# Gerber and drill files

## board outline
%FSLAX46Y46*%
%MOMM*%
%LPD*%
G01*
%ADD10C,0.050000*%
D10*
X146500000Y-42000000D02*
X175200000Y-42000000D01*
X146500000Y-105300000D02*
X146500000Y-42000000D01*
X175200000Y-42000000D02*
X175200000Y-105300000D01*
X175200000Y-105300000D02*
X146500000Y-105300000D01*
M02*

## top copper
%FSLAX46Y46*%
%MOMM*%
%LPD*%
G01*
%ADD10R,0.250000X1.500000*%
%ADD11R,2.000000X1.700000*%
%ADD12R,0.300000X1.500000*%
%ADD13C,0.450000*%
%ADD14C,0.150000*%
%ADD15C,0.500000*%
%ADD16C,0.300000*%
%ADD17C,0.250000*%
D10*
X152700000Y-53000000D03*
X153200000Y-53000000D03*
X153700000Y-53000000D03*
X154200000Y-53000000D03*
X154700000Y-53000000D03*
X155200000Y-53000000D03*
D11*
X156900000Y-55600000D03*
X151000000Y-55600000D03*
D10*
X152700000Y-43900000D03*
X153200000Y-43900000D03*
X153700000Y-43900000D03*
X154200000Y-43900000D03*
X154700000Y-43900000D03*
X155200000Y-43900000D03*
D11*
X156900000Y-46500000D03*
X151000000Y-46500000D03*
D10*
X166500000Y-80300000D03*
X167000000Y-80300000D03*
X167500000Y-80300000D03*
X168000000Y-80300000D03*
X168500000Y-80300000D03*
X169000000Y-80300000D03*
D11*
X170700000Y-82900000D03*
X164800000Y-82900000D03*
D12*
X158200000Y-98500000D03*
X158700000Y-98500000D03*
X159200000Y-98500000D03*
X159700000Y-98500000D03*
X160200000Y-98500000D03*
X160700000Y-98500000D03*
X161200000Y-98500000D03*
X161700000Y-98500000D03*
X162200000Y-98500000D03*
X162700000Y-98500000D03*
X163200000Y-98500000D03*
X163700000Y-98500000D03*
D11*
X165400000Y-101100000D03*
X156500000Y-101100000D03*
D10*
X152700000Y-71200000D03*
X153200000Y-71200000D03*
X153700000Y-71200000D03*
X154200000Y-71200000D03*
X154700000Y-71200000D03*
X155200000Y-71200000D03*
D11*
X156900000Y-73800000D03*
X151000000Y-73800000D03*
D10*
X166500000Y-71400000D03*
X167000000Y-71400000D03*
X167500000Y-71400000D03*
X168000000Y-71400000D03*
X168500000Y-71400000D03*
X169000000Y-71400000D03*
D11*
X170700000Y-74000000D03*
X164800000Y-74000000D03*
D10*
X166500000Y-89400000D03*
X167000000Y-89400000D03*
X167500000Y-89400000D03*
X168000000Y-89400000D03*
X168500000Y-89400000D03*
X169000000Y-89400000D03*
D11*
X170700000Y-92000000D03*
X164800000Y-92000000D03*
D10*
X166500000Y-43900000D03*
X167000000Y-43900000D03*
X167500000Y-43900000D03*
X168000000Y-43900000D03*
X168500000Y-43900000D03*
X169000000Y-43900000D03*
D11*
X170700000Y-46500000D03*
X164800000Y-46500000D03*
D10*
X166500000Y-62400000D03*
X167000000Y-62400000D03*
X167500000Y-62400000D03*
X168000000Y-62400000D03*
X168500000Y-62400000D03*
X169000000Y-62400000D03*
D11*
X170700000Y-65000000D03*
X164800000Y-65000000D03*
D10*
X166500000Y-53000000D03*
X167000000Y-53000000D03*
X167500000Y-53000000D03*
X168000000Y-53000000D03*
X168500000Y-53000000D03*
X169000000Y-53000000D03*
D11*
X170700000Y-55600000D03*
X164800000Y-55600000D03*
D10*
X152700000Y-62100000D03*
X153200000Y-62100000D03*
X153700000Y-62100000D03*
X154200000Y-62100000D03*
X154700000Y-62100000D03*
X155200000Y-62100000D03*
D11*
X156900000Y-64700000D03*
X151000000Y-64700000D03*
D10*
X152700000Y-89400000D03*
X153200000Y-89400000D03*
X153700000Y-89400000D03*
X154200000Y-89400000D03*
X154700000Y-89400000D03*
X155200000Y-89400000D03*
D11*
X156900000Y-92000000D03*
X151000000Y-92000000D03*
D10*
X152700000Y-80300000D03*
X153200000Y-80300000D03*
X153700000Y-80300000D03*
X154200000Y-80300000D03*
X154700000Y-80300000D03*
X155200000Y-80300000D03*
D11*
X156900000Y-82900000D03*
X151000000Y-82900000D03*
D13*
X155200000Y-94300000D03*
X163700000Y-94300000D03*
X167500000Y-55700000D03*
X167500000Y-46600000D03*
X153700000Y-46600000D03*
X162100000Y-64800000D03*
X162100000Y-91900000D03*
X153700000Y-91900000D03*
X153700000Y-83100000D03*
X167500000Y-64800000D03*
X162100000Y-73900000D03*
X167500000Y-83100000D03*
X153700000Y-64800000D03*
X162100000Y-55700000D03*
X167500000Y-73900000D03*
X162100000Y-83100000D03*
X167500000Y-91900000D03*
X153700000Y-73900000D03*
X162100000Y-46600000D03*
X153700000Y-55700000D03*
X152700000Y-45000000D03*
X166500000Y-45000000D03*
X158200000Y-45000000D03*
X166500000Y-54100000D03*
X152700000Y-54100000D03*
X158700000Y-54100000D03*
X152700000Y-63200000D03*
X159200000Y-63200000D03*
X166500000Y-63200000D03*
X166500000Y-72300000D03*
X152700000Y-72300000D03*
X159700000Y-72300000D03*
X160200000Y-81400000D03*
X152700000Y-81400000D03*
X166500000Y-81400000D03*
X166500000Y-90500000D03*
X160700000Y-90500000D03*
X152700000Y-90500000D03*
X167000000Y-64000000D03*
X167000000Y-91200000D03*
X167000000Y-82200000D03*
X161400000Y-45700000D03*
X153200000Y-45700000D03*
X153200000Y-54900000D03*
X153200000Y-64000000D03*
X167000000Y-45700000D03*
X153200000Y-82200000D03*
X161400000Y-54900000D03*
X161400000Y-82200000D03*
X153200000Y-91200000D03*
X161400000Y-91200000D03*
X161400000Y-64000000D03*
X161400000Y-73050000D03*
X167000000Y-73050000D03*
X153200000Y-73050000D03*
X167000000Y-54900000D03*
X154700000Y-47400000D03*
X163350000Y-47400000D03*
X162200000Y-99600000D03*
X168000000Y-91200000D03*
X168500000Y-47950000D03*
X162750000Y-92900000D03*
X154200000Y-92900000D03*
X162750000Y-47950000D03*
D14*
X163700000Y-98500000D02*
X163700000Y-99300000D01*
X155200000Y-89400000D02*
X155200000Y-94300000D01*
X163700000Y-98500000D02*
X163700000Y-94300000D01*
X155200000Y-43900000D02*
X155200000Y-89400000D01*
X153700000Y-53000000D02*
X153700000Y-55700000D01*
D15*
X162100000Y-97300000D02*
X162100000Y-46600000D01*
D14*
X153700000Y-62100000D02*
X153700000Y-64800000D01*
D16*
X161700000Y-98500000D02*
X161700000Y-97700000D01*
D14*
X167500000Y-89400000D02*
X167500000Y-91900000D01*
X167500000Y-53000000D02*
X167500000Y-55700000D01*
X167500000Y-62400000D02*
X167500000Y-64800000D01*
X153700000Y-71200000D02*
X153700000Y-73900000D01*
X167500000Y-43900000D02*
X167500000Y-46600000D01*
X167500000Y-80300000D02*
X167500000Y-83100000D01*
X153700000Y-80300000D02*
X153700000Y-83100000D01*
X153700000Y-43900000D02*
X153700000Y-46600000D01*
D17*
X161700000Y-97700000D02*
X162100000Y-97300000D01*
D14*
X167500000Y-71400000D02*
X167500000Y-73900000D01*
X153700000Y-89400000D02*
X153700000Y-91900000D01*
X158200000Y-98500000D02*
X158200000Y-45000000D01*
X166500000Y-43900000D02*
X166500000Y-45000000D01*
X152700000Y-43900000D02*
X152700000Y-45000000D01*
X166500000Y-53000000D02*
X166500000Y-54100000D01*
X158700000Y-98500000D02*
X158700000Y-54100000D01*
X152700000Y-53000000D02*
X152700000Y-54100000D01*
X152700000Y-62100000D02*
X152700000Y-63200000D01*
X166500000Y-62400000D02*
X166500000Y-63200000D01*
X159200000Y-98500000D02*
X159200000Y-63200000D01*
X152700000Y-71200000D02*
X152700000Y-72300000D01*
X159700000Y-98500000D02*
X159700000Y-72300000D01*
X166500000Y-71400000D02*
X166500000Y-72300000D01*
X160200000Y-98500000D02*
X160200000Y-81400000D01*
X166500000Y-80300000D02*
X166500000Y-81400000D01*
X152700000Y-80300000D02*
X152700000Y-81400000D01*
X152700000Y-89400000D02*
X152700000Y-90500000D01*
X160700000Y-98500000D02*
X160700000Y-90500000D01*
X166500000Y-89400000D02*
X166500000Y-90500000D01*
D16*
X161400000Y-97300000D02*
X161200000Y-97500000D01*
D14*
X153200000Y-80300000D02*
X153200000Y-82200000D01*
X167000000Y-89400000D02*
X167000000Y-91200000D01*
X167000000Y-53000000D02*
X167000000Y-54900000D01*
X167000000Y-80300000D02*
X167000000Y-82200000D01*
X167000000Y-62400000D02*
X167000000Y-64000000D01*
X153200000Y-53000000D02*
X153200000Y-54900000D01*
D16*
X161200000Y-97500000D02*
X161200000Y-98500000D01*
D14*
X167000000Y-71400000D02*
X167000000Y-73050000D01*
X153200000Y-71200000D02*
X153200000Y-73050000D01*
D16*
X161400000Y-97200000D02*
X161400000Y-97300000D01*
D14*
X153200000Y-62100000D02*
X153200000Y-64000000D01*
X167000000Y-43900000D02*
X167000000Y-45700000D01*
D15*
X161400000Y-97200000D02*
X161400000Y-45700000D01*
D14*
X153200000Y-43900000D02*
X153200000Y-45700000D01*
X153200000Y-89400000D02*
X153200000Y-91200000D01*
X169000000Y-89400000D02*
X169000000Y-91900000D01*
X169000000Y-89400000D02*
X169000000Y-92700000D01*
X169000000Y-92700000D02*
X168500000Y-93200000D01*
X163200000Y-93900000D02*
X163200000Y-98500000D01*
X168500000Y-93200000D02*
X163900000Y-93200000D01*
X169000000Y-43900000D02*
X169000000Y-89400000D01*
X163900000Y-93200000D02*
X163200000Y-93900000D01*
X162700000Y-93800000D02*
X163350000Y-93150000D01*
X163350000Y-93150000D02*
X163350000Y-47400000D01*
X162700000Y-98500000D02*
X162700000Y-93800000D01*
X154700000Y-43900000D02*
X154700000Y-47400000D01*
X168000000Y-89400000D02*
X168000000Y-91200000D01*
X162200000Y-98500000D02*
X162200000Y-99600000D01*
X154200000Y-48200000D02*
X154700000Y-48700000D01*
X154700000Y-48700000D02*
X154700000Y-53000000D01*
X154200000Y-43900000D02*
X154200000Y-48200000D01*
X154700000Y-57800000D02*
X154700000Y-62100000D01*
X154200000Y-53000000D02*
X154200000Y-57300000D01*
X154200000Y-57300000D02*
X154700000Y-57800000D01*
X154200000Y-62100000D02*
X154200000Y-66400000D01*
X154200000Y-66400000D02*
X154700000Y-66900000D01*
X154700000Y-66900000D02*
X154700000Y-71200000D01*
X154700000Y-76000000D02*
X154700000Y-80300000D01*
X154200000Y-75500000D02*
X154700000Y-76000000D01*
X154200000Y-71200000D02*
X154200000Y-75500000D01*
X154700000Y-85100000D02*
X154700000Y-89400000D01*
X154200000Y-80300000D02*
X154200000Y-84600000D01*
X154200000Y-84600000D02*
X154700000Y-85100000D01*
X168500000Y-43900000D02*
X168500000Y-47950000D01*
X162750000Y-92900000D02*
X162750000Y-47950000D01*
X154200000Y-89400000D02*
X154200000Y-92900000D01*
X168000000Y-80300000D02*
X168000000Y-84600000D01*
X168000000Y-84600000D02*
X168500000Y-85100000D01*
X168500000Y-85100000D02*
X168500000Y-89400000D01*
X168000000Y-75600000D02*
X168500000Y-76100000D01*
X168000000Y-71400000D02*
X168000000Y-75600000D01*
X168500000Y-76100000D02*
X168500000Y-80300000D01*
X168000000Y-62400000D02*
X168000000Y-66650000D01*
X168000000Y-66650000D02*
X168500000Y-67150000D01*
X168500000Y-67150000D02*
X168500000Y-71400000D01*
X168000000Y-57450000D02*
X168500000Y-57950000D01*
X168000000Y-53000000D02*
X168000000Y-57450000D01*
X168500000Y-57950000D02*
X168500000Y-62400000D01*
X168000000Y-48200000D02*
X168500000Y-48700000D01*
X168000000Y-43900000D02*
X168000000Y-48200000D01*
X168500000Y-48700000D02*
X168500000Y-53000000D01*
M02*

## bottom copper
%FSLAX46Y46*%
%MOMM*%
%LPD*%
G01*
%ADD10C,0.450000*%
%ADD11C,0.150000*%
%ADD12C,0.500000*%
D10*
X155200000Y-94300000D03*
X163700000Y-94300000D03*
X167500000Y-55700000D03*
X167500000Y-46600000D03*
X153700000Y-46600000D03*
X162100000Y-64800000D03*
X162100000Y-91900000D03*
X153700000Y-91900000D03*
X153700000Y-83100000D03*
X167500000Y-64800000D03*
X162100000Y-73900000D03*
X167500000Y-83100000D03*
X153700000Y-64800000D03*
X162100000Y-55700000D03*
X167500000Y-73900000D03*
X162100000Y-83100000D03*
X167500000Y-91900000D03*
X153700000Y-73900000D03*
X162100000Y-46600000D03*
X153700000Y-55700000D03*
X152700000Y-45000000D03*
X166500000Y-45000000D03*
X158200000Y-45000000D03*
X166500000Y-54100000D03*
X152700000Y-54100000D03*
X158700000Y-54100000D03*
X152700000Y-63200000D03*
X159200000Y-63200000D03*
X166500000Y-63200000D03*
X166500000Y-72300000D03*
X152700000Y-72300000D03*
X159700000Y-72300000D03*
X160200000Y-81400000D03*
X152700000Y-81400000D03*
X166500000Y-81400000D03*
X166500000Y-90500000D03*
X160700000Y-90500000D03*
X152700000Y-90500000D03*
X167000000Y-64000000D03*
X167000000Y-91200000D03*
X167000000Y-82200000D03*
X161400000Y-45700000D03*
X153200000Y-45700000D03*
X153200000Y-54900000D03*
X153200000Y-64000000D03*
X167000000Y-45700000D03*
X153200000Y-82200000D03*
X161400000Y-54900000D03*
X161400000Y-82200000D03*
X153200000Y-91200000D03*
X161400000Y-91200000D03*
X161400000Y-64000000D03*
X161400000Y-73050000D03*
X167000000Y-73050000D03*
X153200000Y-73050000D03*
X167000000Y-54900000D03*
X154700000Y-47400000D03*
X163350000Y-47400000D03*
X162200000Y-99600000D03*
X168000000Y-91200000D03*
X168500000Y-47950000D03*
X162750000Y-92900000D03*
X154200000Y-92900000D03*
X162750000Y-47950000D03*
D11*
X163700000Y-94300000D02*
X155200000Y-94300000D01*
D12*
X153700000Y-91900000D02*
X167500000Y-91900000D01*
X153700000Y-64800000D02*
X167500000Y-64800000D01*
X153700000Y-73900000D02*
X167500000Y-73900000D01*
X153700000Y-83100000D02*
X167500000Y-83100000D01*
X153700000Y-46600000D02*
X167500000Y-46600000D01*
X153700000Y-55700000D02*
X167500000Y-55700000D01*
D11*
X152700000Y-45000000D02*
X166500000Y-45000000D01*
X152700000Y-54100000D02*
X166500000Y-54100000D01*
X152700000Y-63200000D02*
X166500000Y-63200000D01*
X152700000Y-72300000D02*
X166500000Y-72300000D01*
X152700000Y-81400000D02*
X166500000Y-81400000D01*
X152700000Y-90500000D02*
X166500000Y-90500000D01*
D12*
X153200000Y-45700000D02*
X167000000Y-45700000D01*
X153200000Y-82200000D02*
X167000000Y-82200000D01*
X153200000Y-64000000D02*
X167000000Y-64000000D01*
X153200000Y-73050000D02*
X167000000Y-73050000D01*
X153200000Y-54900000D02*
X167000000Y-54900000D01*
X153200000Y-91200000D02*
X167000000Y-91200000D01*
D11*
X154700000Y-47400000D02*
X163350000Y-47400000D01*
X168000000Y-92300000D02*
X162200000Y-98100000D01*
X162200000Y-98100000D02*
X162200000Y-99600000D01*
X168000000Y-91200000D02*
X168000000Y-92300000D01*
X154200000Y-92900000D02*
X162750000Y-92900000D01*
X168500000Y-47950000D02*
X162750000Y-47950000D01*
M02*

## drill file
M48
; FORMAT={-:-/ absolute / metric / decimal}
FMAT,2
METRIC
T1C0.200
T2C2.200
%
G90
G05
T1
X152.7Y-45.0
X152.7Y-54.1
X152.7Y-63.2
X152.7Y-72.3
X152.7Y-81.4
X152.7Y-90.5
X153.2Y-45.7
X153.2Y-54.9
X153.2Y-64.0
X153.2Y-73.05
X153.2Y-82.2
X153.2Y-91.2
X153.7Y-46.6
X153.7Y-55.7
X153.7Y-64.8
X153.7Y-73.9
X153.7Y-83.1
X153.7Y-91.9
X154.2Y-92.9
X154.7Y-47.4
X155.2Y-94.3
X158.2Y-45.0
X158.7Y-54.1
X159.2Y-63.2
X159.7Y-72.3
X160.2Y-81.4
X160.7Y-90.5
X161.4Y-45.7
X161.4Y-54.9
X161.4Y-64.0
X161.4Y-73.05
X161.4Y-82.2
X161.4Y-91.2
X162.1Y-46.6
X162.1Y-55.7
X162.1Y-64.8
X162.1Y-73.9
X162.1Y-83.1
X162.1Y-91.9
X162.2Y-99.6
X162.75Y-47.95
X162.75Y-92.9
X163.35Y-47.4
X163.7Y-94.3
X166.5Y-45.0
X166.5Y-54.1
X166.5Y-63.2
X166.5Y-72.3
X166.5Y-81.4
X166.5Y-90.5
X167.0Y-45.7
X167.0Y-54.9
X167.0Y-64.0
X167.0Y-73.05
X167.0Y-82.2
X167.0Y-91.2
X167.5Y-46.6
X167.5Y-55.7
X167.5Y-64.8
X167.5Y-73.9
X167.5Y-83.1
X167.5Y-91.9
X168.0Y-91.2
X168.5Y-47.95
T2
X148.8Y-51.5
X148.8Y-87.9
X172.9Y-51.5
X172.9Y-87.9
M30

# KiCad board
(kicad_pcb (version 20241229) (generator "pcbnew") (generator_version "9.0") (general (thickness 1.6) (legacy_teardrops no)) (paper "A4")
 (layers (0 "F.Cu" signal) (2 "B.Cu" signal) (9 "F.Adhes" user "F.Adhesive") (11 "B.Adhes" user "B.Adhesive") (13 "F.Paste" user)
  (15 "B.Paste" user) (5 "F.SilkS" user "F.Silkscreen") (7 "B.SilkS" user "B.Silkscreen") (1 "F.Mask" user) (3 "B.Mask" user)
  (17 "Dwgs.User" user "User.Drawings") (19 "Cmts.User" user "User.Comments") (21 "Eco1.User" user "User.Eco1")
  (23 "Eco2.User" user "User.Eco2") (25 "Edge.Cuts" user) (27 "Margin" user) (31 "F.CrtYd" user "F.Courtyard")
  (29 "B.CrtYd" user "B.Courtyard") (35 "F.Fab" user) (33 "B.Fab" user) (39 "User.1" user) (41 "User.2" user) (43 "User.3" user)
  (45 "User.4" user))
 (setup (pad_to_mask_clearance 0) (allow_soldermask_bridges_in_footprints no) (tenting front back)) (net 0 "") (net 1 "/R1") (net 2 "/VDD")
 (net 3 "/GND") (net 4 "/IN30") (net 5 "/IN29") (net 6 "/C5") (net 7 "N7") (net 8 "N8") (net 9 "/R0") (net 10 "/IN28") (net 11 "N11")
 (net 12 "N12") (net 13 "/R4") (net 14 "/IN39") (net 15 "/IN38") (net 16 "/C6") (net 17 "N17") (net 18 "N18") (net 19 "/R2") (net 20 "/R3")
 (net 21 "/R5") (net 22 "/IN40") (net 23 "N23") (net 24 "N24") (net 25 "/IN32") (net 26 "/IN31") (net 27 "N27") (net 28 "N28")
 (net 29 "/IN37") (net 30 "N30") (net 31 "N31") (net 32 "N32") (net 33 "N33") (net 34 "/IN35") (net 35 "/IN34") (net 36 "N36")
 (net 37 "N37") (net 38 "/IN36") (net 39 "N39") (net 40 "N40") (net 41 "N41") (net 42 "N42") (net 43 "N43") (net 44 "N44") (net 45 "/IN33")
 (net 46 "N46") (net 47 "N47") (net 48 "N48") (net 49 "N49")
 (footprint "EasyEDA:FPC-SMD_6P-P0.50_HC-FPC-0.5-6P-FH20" (layer "F.Cu") (at 153.95 54.3)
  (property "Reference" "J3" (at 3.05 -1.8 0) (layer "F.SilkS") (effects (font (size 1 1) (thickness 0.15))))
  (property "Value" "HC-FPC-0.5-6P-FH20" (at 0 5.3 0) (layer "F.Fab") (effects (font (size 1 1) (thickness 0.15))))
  (pad "1" smd rect (at -1.25 -1.3) (size 0.25 1.5) (layers "F.Cu" "F.Mask" "F.Paste") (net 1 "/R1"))
  (pad "2" smd rect (at -0.75 -1.3) (size 0.25 1.5) (layers "F.Cu" "F.Mask" "F.Paste") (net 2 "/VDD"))
  (pad "3" smd rect (at -0.25 -1.3) (size 0.25 1.5) (layers "F.Cu" "F.Mask" "F.Paste") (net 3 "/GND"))
  (pad "4" smd rect (at 0.25 -1.3) (size 0.25 1.5) (layers "F.Cu" "F.Mask" "F.Paste") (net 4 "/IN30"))
  (pad "5" smd rect (at 0.75 -1.3) (size 0.25 1.5) (layers "F.Cu" "F.Mask" "F.Paste") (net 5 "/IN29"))
  (pad "6" smd rect (at 1.25 -1.3) (size 0.25 1.5) (layers "F.Cu" "F.Mask" "F.Paste") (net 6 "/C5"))
  (pad "7" smd rect (at 2.95 1.3) (size 2 1.7) (layers "F.Cu" "F.Mask" "F.Paste") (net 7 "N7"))
  (pad "8" smd rect (at -2.95 1.3) (size 2 1.7) (layers "F.Cu" "F.Mask" "F.Paste") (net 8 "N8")))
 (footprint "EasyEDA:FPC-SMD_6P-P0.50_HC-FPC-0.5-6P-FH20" (layer "F.Cu") (at 153.95 45.2)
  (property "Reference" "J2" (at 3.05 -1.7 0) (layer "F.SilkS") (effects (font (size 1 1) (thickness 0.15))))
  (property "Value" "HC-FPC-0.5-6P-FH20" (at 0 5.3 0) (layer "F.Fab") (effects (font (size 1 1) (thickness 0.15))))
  (pad "1" smd rect (at -1.25 -1.3) (size 0.25 1.5) (layers "F.Cu" "F.Mask" "F.Paste") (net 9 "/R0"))
  (pad "2" smd rect (at -0.75 -1.3) (size 0.25 1.5) (layers "F.Cu" "F.Mask" "F.Paste") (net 2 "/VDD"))
  (pad "3" smd rect (at -0.25 -1.3) (size 0.25 1.5) (layers "F.Cu" "F.Mask" "F.Paste") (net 3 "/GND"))
  (pad "4" smd rect (at 0.25 -1.3) (size 0.25 1.5) (layers "F.Cu" "F.Mask" "F.Paste") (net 5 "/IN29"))
  (pad "5" smd rect (at 0.75 -1.3) (size 0.25 1.5) (layers "F.Cu" "F.Mask" "F.Paste") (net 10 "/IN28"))
  (pad "6" smd rect (at 1.25 -1.3) (size 0.25 1.5) (layers "F.Cu" "F.Mask" "F.Paste") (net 6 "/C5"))
  (pad "7" smd rect (at 2.95 1.3) (size 2 1.7) (layers "F.Cu" "F.Mask" "F.Paste") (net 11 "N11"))
  (pad "8" smd rect (at -2.95 1.3) (size 2 1.7) (layers "F.Cu" "F.Mask" "F.Paste") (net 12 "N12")))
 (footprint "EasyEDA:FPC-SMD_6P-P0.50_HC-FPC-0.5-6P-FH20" (layer "F.Cu") (at 167.75 81.6)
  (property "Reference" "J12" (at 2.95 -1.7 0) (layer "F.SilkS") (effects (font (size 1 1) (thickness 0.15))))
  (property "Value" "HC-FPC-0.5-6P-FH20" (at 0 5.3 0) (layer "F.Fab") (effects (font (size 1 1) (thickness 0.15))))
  (pad "1" smd rect (at -1.25 -1.3) (size 0.25 1.5) (layers "F.Cu" "F.Mask" "F.Paste") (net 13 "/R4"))
  (pad "2" smd rect (at -0.75 -1.3) (size 0.25 1.5) (layers "F.Cu" "F.Mask" "F.Paste") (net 2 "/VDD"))
  (pad "3" smd rect (at -0.25 -1.3) (size 0.25 1.5) (layers "F.Cu" "F.Mask" "F.Paste") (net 3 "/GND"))
  (pad "4" smd rect (at 0.25 -1.3) (size 0.25 1.5) (layers "F.Cu" "F.Mask" "F.Paste") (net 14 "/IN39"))
  (pad "5" smd rect (at 0.75 -1.3) (size 0.25 1.5) (layers "F.Cu" "F.Mask" "F.Paste") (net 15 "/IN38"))
  (pad "6" smd rect (at 1.25 -1.3) (size 0.25 1.5) (layers "F.Cu" "F.Mask" "F.Paste") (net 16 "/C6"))
  (pad "7" smd rect (at 2.95 1.3) (size 2 1.7) (layers "F.Cu" "F.Mask" "F.Paste") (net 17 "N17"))
  (pad "8" smd rect (at -2.95 1.3) (size 2 1.7) (layers "F.Cu" "F.Mask" "F.Paste") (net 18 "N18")))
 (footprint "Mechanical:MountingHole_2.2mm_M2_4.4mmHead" (layer "F.Cu") (at 148.8 87.9)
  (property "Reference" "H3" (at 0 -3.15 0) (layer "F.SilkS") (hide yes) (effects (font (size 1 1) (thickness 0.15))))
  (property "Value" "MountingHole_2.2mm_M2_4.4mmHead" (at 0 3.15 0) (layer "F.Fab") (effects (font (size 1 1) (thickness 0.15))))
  (pad "" np_thru_hole circle (at 0 0) (size 2.2 2.2) (drill 2.2) (layers "*.Cu" "*.Mask")))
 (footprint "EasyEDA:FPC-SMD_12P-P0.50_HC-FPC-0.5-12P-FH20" (layer "F.Cu") (at 160.95 99.8)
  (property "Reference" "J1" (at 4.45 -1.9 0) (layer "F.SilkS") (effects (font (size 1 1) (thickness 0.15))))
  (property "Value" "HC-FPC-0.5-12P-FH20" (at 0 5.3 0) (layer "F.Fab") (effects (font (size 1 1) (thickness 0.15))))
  (pad "1" smd rect (at -2.75 -1.3) (size 0.3 1.5) (layers "F.Cu" "F.Mask" "F.Paste") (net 9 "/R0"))
  (pad "2" smd rect (at -2.25 -1.3) (size 0.3 1.5) (layers "F.Cu" "F.Mask" "F.Paste") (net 1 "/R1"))
  (pad "3" smd rect (at -1.75 -1.3) (size 0.3 1.5) (layers "F.Cu" "F.Mask" "F.Paste") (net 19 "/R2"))
  (pad "4" smd rect (at -1.25 -1.3) (size 0.3 1.5) (layers "F.Cu" "F.Mask" "F.Paste") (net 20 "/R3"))
  (pad "5" smd rect (at -0.75 -1.3) (size 0.3 1.5) (layers "F.Cu" "F.Mask" "F.Paste") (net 13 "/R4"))
  (pad "6" smd rect (at -0.25 -1.3) (size 0.3 1.5) (layers "F.Cu" "F.Mask" "F.Paste") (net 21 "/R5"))
  (pad "7" smd rect (at 0.25 -1.3) (size 0.3 1.5) (layers "F.Cu" "F.Mask" "F.Paste") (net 2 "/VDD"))
  (pad "8" smd rect (at 0.75 -1.3) (size 0.3 1.5) (layers "F.Cu" "F.Mask" "F.Paste") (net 3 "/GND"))
  (pad "9" smd rect (at 1.25 -1.3) (size 0.3 1.5) (layers "F.Cu" "F.Mask" "F.Paste") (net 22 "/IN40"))
  (pad "10" smd rect (at 1.75 -1.3) (size 0.3 1.5) (layers "F.Cu" "F.Mask" "F.Paste") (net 10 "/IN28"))
  (pad "11" smd rect (at 2.25 -1.3) (size 0.3 1.5) (layers "F.Cu" "F.Mask" "F.Paste") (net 16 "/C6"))
  (pad "12" smd rect (at 2.75 -1.3) (size 0.3 1.5) (layers "F.Cu" "F.Mask" "F.Paste") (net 6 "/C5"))
  (pad "13" smd rect (at 4.45 1.3) (size 2 1.7) (layers "F.Cu" "F.Mask" "F.Paste") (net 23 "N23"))
  (pad "14" smd rect (at -4.45 1.3) (size 2 1.7) (layers "F.Cu" "F.Mask" "F.Paste") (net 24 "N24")))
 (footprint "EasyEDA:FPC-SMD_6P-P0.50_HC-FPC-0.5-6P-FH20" (layer "F.Cu") (at 153.95 72.5)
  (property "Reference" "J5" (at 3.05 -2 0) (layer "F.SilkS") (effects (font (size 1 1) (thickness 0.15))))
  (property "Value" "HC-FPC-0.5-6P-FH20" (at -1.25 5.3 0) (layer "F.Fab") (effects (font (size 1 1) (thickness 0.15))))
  (pad "1" smd rect (at -1.25 -1.3) (size 0.25 1.5) (layers "F.Cu" "F.Mask" "F.Paste") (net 20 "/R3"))
  (pad "2" smd rect (at -0.75 -1.3) (size 0.25 1.5) (layers "F.Cu" "F.Mask" "F.Paste") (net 2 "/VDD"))
  (pad "3" smd rect (at -0.25 -1.3) (size 0.25 1.5) (layers "F.Cu" "F.Mask" "F.Paste") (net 3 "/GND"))
  (pad "4" smd rect (at 0.25 -1.3) (size 0.25 1.5) (layers "F.Cu" "F.Mask" "F.Paste") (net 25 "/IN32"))
  (pad "5" smd rect (at 0.75 -1.3) (size 0.25 1.5) (layers "F.Cu" "F.Mask" "F.Paste") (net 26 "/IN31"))
  (pad "6" smd rect (at 1.25 -1.3) (size 0.25 1.5) (layers "F.Cu" "F.Mask" "F.Paste") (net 6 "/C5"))
  (pad "7" smd rect (at 2.95 1.3) (size 2 1.7) (layers "F.Cu" "F.Mask" "F.Paste") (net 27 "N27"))
  (pad "8" smd rect (at -2.95 1.3) (size 2 1.7) (layers "F.Cu" "F.Mask" "F.Paste") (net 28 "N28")))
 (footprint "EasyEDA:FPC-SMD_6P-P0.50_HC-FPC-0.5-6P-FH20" (layer "F.Cu") (at 167.75 72.7)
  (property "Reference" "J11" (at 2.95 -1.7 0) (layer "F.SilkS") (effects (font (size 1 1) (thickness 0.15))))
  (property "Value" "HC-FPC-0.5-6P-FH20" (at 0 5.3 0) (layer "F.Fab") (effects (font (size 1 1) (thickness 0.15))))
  (pad "1" smd rect (at -1.25 -1.3) (size 0.25 1.5) (layers "F.Cu" "F.Mask" "F.Paste") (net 20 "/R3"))
  (pad "2" smd rect (at -0.75 -1.3) (size 0.25 1.5) (layers "F.Cu" "F.Mask" "F.Paste") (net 2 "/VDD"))
  (pad "3" smd rect (at -0.25 -1.3) (size 0.25 1.5) (layers "F.Cu" "F.Mask" "F.Paste") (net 3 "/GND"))
  (pad "4" smd rect (at 0.25 -1.3) (size 0.25 1.5) (layers "F.Cu" "F.Mask" "F.Paste") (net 15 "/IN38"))
  (pad "5" smd rect (at 0.75 -1.3) (size 0.25 1.5) (layers "F.Cu" "F.Mask" "F.Paste") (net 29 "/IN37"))
  (pad "6" smd rect (at 1.25 -1.3) (size 0.25 1.5) (layers "F.Cu" "F.Mask" "F.Paste") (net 16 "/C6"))
  (pad "7" smd rect (at 2.95 1.3) (size 2 1.7) (layers "F.Cu" "F.Mask" "F.Paste") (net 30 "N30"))
  (pad "8" smd rect (at -2.95 1.3) (size 2 1.7) (layers "F.Cu" "F.Mask" "F.Paste") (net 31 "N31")))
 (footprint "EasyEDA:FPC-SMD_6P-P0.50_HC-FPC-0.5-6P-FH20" (layer "F.Cu") (at 167.75 90.7)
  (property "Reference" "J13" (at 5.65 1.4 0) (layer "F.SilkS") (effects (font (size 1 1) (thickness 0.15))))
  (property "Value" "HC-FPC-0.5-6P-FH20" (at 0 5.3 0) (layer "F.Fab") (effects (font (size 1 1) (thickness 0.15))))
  (pad "1" smd rect (at -1.25 -1.3) (size 0.25 1.5) (layers "F.Cu" "F.Mask" "F.Paste") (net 21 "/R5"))
  (pad "2" smd rect (at -0.75 -1.3) (size 0.25 1.5) (layers "F.Cu" "F.Mask" "F.Paste") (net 2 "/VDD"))
  (pad "3" smd rect (at -0.25 -1.3) (size 0.25 1.5) (layers "F.Cu" "F.Mask" "F.Paste") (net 3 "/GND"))
  (pad "4" smd rect (at 0.25 -1.3) (size 0.25 1.5) (layers "F.Cu" "F.Mask" "F.Paste") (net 22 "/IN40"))
  (pad "5" smd rect (at 0.75 -1.3) (size 0.25 1.5) (layers "F.Cu" "F.Mask" "F.Paste") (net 14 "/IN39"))
  (pad "6" smd rect (at 1.25 -1.3) (size 0.25 1.5) (layers "F.Cu" "F.Mask" "F.Paste") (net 16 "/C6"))
  (pad "7" smd rect (at 2.95 1.3) (size 2 1.7) (layers "F.Cu" "F.Mask" "F.Paste") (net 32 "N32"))
  (pad "8" smd rect (at -2.95 1.3) (size 2 1.7) (layers "F.Cu" "F.Mask" "F.Paste") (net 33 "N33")))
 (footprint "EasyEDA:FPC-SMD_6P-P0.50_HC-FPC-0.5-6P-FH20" (layer "F.Cu") (at 167.75 45.2)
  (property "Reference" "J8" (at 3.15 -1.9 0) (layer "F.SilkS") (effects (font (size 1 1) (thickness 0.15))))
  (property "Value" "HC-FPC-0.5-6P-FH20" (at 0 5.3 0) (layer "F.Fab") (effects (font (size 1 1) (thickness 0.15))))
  (pad "1" smd rect (at -1.25 -1.3) (size 0.25 1.5) (layers "F.Cu" "F.Mask" "F.Paste") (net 9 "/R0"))
  (pad "2" smd rect (at -0.75 -1.3) (size 0.25 1.5) (layers "F.Cu" "F.Mask" "F.Paste") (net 2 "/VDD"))
  (pad "3" smd rect (at -0.25 -1.3) (size 0.25 1.5) (layers "F.Cu" "F.Mask" "F.Paste") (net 3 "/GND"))
  (pad "4" smd rect (at 0.25 -1.3) (size 0.25 1.5) (layers "F.Cu" "F.Mask" "F.Paste") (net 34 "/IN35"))
  (pad "5" smd rect (at 0.75 -1.3) (size 0.25 1.5) (layers "F.Cu" "F.Mask" "F.Paste") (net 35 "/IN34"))
  (pad "6" smd rect (at 1.25 -1.3) (size 0.25 1.5) (layers "F.Cu" "F.Mask" "F.Paste") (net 16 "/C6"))
  (pad "7" smd rect (at 2.95 1.3) (size 2 1.7) (layers "F.Cu" "F.Mask" "F.Paste") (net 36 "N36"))
  (pad "8" smd rect (at -2.95 1.3) (size 2 1.7) (layers "F.Cu" "F.Mask" "F.Paste") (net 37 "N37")))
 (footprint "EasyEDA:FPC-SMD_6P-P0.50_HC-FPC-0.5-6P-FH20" (layer "F.Cu") (at 167.75 63.7)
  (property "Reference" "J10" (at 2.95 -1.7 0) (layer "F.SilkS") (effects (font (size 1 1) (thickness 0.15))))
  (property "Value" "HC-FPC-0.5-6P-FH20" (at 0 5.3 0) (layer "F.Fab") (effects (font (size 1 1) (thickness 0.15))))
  (pad "1" smd rect (at -1.25 -1.3) (size 0.25 1.5) (layers "F.Cu" "F.Mask" "F.Paste") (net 19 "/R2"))
  (pad "2" smd rect (at -0.75 -1.3) (size 0.25 1.5) (layers "F.Cu" "F.Mask" "F.Paste") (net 2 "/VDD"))
  (pad "3" smd rect (at -0.25 -1.3) (size 0.25 1.5) (layers "F.Cu" "F.Mask" "F.Paste") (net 3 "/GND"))
  (pad "4" smd rect (at 0.25 -1.3) (size 0.25 1.5) (layers "F.Cu" "F.Mask" "F.Paste") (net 29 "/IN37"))
  (pad "5" smd rect (at 0.75 -1.3) (size 0.25 1.5) (layers "F.Cu" "F.Mask" "F.Paste") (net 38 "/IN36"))
  (pad "6" smd rect (at 1.25 -1.3) (size 0.25 1.5) (layers "F.Cu" "F.Mask" "F.Paste") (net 16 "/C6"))
  (pad "7" smd rect (at 2.95 1.3) (size 2 1.7) (layers "F.Cu" "F.Mask" "F.Paste") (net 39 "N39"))
  (pad "8" smd rect (at -2.95 1.3) (size 2 1.7) (layers "F.Cu" "F.Mask" "F.Paste") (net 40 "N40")))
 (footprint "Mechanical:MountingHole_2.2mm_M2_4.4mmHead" (layer "F.Cu") (at 172.9 51.5)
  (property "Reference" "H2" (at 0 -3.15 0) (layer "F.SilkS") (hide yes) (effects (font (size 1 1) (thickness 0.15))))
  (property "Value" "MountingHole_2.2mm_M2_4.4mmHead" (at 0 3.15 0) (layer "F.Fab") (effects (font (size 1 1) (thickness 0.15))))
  (pad "" np_thru_hole circle (at 0 0) (size 2.2 2.2) (drill 2.2) (layers "*.Cu" "*.Mask")))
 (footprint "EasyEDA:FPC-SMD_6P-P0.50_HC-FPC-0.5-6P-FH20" (layer "F.Cu") (at 167.75 54.3)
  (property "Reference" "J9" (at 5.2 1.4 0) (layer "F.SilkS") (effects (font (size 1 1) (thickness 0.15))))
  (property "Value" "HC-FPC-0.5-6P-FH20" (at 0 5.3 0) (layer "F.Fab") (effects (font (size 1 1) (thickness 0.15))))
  (pad "1" smd rect (at -1.25 -1.3) (size 0.25 1.5) (layers "F.Cu" "F.Mask" "F.Paste") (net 1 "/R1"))
  (pad "2" smd rect (at -0.75 -1.3) (size 0.25 1.5) (layers "F.Cu" "F.Mask" "F.Paste") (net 2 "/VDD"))
  (pad "3" smd rect (at -0.25 -1.3) (size 0.25 1.5) (layers "F.Cu" "F.Mask" "F.Paste") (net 3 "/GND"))
  (pad "4" smd rect (at 0.25 -1.3) (size 0.25 1.5) (layers "F.Cu" "F.Mask" "F.Paste") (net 38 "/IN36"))
  (pad "5" smd rect (at 0.75 -1.3) (size 0.25 1.5) (layers "F.Cu" "F.Mask" "F.Paste") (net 34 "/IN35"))
  (pad "6" smd rect (at 1.25 -1.3) (size 0.25 1.5) (layers "F.Cu" "F.Mask" "F.Paste") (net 16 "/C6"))
  (pad "7" smd rect (at 2.95 1.3) (size 2 1.7) (layers "F.Cu" "F.Mask" "F.Paste") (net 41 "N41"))
  (pad "8" smd rect (at -2.95 1.3) (size 2 1.7) (layers "F.Cu" "F.Mask" "F.Paste") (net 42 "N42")))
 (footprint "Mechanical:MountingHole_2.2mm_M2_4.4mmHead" (layer "F.Cu") (at 148.8 51.5)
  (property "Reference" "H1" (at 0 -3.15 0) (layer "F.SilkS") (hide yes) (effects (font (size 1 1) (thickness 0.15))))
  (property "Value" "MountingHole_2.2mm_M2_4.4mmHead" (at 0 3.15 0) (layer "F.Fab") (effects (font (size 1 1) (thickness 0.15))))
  (pad "" np_thru_hole circle (at 0 0) (size 2.2 2.2) (drill 2.2) (layers "*.Cu" "*.Mask")))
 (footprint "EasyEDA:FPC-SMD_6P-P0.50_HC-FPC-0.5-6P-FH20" (layer "F.Cu") (at 153.95 63.4)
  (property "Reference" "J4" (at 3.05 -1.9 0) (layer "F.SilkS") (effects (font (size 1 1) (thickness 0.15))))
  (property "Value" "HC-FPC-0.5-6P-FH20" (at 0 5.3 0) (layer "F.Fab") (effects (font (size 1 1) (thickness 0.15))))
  (pad "1" smd rect (at -1.25 -1.3) (size 0.25 1.5) (layers "F.Cu" "F.Mask" "F.Paste") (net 19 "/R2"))
  (pad "2" smd rect (at -0.75 -1.3) (size 0.25 1.5) (layers "F.Cu" "F.Mask" "F.Paste") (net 2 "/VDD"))
  (pad "3" smd rect (at -0.25 -1.3) (size 0.25 1.5) (layers "F.Cu" "F.Mask" "F.Paste") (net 3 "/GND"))
  (pad "4" smd rect (at 0.25 -1.3) (size 0.25 1.5) (layers "F.Cu" "F.Mask" "F.Paste") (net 26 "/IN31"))
  (pad "5" smd rect (at 0.75 -1.3) (size 0.25 1.5) (layers "F.Cu" "F.Mask" "F.Paste") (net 4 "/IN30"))
  (pad "6" smd rect (at 1.25 -1.3) (size 0.25 1.5) (layers "F.Cu" "F.Mask" "F.Paste") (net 6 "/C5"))
  (pad "7" smd rect (at 2.95 1.3) (size 2 1.7) (layers "F.Cu" "F.Mask" "F.Paste") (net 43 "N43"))
  (pad "8" smd rect (at -2.95 1.3) (size 2 1.7) (layers "F.Cu" "F.Mask" "F.Paste") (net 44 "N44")))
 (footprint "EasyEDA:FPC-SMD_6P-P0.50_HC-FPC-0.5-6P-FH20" (layer "F.Cu") (at 153.95 90.7)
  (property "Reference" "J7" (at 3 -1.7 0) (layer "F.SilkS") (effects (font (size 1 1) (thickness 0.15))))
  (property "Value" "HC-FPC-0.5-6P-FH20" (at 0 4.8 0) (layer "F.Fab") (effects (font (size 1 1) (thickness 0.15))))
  (pad "1" smd rect (at -1.25 -1.3) (size 0.25 1.5) (layers "F.Cu" "F.Mask" "F.Paste") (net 21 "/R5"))
  (pad "2" smd rect (at -0.75 -1.3) (size 0.25 1.5) (layers "F.Cu" "F.Mask" "F.Paste") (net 2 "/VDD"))
  (pad "3" smd rect (at -0.25 -1.3) (size 0.25 1.5) (layers "F.Cu" "F.Mask" "F.Paste") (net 3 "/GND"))
  (pad "4" smd rect (at 0.25 -1.3) (size 0.25 1.5) (layers "F.Cu" "F.Mask" "F.Paste") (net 35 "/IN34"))
  (pad "5" smd rect (at 0.75 -1.3) (size 0.25 1.5) (layers "F.Cu" "F.Mask" "F.Paste") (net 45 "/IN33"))
  (pad "6" smd rect (at 1.25 -1.3) (size 0.25 1.5) (layers "F.Cu" "F.Mask" "F.Paste") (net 6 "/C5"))
  (pad "7" smd rect (at 2.95 1.3) (size 2 1.7) (layers "F.Cu" "F.Mask" "F.Paste") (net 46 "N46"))
  (pad "8" smd rect (at -2.95 1.3) (size 2 1.7) (layers "F.Cu" "F.Mask" "F.Paste") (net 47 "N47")))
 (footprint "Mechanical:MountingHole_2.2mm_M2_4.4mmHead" (layer "F.Cu") (at 172.9 87.9)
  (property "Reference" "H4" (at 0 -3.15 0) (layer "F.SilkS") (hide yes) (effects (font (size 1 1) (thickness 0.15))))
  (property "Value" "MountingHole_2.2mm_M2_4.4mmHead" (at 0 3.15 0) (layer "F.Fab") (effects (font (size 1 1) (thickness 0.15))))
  (pad "" np_thru_hole circle (at 0 0) (size 2.2 2.2) (drill 2.2) (layers "*.Cu" "*.Mask")))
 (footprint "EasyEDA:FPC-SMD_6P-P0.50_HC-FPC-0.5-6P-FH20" (layer "F.Cu") (at 153.95 81.6)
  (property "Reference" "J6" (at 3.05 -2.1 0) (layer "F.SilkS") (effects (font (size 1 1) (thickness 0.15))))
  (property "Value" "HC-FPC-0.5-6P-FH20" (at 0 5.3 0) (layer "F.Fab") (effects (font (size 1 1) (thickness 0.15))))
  (pad "1" smd rect (at -1.25 -1.3) (size 0.25 1.5) (layers "F.Cu" "F.Mask" "F.Paste") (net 13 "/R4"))
  (pad "2" smd rect (at -0.75 -1.3) (size 0.25 1.5) (layers "F.Cu" "F.Mask" "F.Paste") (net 2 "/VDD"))
  (pad "3" smd rect (at -0.25 -1.3) (size 0.25 1.5) (layers "F.Cu" "F.Mask" "F.Paste") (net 3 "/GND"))
  (pad "4" smd rect (at 0.25 -1.3) (size 0.25 1.5) (layers "F.Cu" "F.Mask" "F.Paste") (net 45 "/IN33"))
  (pad "5" smd rect (at 0.75 -1.3) (size 0.25 1.5) (layers "F.Cu" "F.Mask" "F.Paste") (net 25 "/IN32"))
  (pad "6" smd rect (at 1.25 -1.3) (size 0.25 1.5) (layers "F.Cu" "F.Mask" "F.Paste") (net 6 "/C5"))
  (pad "7" smd rect (at 2.95 1.3) (size 2 1.7) (layers "F.Cu" "F.Mask" "F.Paste") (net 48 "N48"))
  (pad "8" smd rect (at -2.95 1.3) (size 2 1.7) (layers "F.Cu" "F.Mask" "F.Paste") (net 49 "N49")))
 (gr_line (start 146.5 42) (end 175.2 42) (stroke (width 0.05) (type default)) (layer "Edge.Cuts"))
 (gr_line (start 146.5 105.3) (end 146.5 42) (stroke (width 0.05) (type default)) (layer "Edge.Cuts"))
 (gr_line (start 175.2 42) (end 175.2 105.3) (stroke (width 0.05) (type default)) (layer "Edge.Cuts"))
 (gr_line (start 175.2 105.3) (end 146.5 105.3) (stroke (width 0.05) (type default)) (layer "Edge.Cuts"))
 (segment (start 163.7 98.5) (end 163.7 99.3) (width 0.15) (layer "F.Cu") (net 6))
 (segment (start 155.2 89.4) (end 155.2 94.3) (width 0.15) (layer "F.Cu") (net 6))
 (segment (start 163.7 98.5) (end 163.7 94.3) (width 0.15) (layer "F.Cu") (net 6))
 (segment (start 155.2 43.9) (end 155.2 89.4) (width 0.15) (layer "F.Cu") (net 6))
 (via (at 155.2 94.3) (size 0.45) (drill 0.2) (layers "F.Cu" "B.Cu") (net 6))
 (via (at 163.7 94.3) (size 0.45) (drill 0.2) (layers "F.Cu" "B.Cu") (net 6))
 (segment (start 163.7 94.3) (end 155.2 94.3) (width 0.15) (layer "B.Cu") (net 6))
 (segment (start 153.7 53) (end 153.7 55.7) (width 0.15) (layer "F.Cu") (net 3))
 (segment (start 162.1 97.3) (end 162.1 46.6) (width 0.5) (layer "F.Cu") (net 3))
 (segment (start 153.7 62.1) (end 153.7 64.8) (width 0.15) (layer "F.Cu") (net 3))
 (segment (start 161.7 98.5) (end 161.7 97.7) (width 0.3) (layer "F.Cu") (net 3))
 (segment (start 167.5 89.4) (end 167.5 91.9) (width 0.15) (layer "F.Cu") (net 3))
 (segment (start 167.5 53) (end 167.5 55.7) (width 0.15) (layer "F.Cu") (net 3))
 (segment (start 167.5 62.4) (end 167.5 64.8) (width 0.15) (layer "F.Cu") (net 3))
 (segment (start 153.7 71.2) (end 153.7 73.9) (width 0.15) (layer "F.Cu") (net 3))
 (segment (start 167.5 43.9) (end 167.5 46.6) (width 0.15) (layer "F.Cu") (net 3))
 (segment (start 167.5 80.3) (end 167.5 83.1) (width 0.15) (layer "F.Cu") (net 3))
 (segment (start 153.7 80.3) (end 153.7 83.1) (width 0.15) (layer "F.Cu") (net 3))
 (segment (start 153.7 43.9) (end 153.7 46.6) (width 0.15) (layer "F.Cu") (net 3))
 (segment (start 161.7 97.7) (end 162.1 97.3) (width 0.25) (layer "F.Cu") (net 3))
 (segment (start 167.5 71.4) (end 167.5 73.9) (width 0.15) (layer "F.Cu") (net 3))
 (segment (start 153.7 89.4) (end 153.7 91.9) (width 0.15) (layer "F.Cu") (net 3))
 (via (at 167.5 55.7) (size 0.45) (drill 0.2) (layers "F.Cu" "B.Cu") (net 3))
 (via (at 167.5 46.6) (size 0.45) (drill 0.2) (layers "F.Cu" "B.Cu") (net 3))
 (via (at 153.7 46.6) (size 0.45) (drill 0.2) (layers "F.Cu" "B.Cu") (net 3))
 (via (at 162.1 64.8) (size 0.45) (drill 0.2) (layers "F.Cu" "B.Cu") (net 3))
 (via (at 162.1 91.9) (size 0.45) (drill 0.2) (layers "F.Cu" "B.Cu") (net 3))
 (via (at 153.7 91.9) (size 0.45) (drill 0.2) (layers "F.Cu" "B.Cu") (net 3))
 (via (at 153.7 83.1) (size 0.45) (drill 0.2) (layers "F.Cu" "B.Cu") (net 3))
 (via (at 167.5 64.8) (size 0.45) (drill 0.2) (layers "F.Cu" "B.Cu") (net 3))
 (via (at 162.1 73.9) (size 0.45) (drill 0.2) (layers "F.Cu" "B.Cu") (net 3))
 (via (at 167.5 83.1) (size 0.45) (drill 0.2) (layers "F.Cu" "B.Cu") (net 3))
 (via (at 153.7 64.8) (size 0.45) (drill 0.2) (layers "F.Cu" "B.Cu") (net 3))
 (via (at 162.1 55.7) (size 0.45) (drill 0.2) (layers "F.Cu" "B.Cu") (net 3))
 (via (at 167.5 73.9) (size 0.45) (drill 0.2) (layers "F.Cu" "B.Cu") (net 3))
 (via (at 162.1 83.1) (size 0.45) (drill 0.2) (layers "F.Cu" "B.Cu") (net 3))
 (via (at 167.5 91.9) (size 0.45) (drill 0.2) (layers "F.Cu" "B.Cu") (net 3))
 (via (at 153.7 73.9) (size 0.45) (drill 0.2) (layers "F.Cu" "B.Cu") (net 3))
 (via (at 162.1 46.6) (size 0.45) (drill 0.2) (layers "F.Cu" "B.Cu") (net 3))
 (via (at 153.7 55.7) (size 0.45) (drill 0.2) (layers "F.Cu" "B.Cu") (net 3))
 (segment (start 153.7 91.9) (end 167.5 91.9) (width 0.5) (layer "B.Cu") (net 3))
 (segment (start 153.7 64.8) (end 167.5 64.8) (width 0.5) (layer "B.Cu") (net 3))
 (segment (start 153.7 73.9) (end 167.5 73.9) (width 0.5) (layer "B.Cu") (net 3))
 (segment (start 153.7 83.1) (end 167.5 83.1) (width 0.5) (layer "B.Cu") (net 3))
 (segment (start 153.7 46.6) (end 167.5 46.6) (width 0.5) (layer "B.Cu") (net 3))
 (segment (start 153.7 55.7) (end 167.5 55.7) (width 0.5) (layer "B.Cu") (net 3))
 (segment (start 158.2 98.5) (end 158.2 45) (width 0.15) (layer "F.Cu") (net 9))
 (segment (start 166.5 43.9) (end 166.5 45) (width 0.15) (layer "F.Cu") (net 9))
 (segment (start 152.7 43.9) (end 152.7 45) (width 0.15) (layer "F.Cu") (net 9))
 (via (at 152.7 45) (size 0.45) (drill 0.2) (layers "F.Cu" "B.Cu") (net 9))
 (via (at 166.5 45) (size 0.45) (drill 0.2) (layers "F.Cu" "B.Cu") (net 9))
 (via (at 158.2 45) (size 0.45) (drill 0.2) (layers "F.Cu" "B.Cu") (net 9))
 (segment (start 152.7 45) (end 166.5 45) (width 0.15) (layer "B.Cu") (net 9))
 (segment (start 166.5 53) (end 166.5 54.1) (width 0.15) (layer "F.Cu") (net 1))
 (segment (start 158.7 98.5) (end 158.7 54.1) (width 0.15) (layer "F.Cu") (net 1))
 (segment (start 152.7 53) (end 152.7 54.1) (width 0.15) (layer "F.Cu") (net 1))
 (via (at 166.5 54.1) (size 0.45) (drill 0.2) (layers "F.Cu" "B.Cu") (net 1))
 (via (at 152.7 54.1) (size 0.45) (drill 0.2) (layers "F.Cu" "B.Cu") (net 1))
 (via (at 158.7 54.1) (size 0.45) (drill 0.2) (layers "F.Cu" "B.Cu") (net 1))
 (segment (start 152.7 54.1) (end 166.5 54.1) (width 0.15) (layer "B.Cu") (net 1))
 (segment (start 152.7 62.1) (end 152.7 63.2) (width 0.15) (layer "F.Cu") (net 19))
 (segment (start 166.5 62.4) (end 166.5 63.2) (width 0.15) (layer "F.Cu") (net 19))
 (segment (start 159.2 98.5) (end 159.2 63.2) (width 0.15) (layer "F.Cu") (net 19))
 (via (at 152.7 63.2) (size 0.45) (drill 0.2) (layers "F.Cu" "B.Cu") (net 19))
 (via (at 159.2 63.2) (size 0.45) (drill 0.2) (layers "F.Cu" "B.Cu") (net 19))
 (via (at 166.5 63.2) (size 0.45) (drill 0.2) (layers "F.Cu" "B.Cu") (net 19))
 (segment (start 152.7 63.2) (end 166.5 63.2) (width 0.15) (layer "B.Cu") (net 19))
 (segment (start 152.7 71.2) (end 152.7 72.3) (width 0.15) (layer "F.Cu") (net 20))
 (segment (start 159.7 98.5) (end 159.7 72.3) (width 0.15) (layer "F.Cu") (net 20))
 (segment (start 166.5 71.4) (end 166.5 72.3) (width 0.15) (layer "F.Cu") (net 20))
 (via (at 166.5 72.3) (size 0.45) (drill 0.2) (layers "F.Cu" "B.Cu") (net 20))
 (via (at 152.7 72.3) (size 0.45) (drill 0.2) (layers "F.Cu" "B.Cu") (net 20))
 (via (at 159.7 72.3) (size 0.45) (drill 0.2) (layers "F.Cu" "B.Cu") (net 20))
 (segment (start 152.7 72.3) (end 166.5 72.3) (width 0.15) (layer "B.Cu") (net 20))
 (segment (start 160.2 98.5) (end 160.2 81.4) (width 0.15) (layer "F.Cu") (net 13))
 (segment (start 166.5 80.3) (end 166.5 81.4) (width 0.15) (layer "F.Cu") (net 13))
 (segment (start 152.7 80.3) (end 152.7 81.4) (width 0.15) (layer "F.Cu") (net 13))
 (via (at 160.2 81.4) (size 0.45) (drill 0.2) (layers "F.Cu" "B.Cu") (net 13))
 (via (at 152.7 81.4) (size 0.45) (drill 0.2) (layers "F.Cu" "B.Cu") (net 13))
 (via (at 166.5 81.4) (size 0.45) (drill 0.2) (layers "F.Cu" "B.Cu") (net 13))
 (segment (start 152.7 81.4) (end 166.5 81.4) (width 0.15) (layer "B.Cu") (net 13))
 (segment (start 152.7 89.4) (end 152.7 90.5) (width 0.15) (layer "F.Cu") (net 21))
 (segment (start 160.7 98.5) (end 160.7 90.5) (width 0.15) (layer "F.Cu") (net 21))
 (segment (start 166.5 89.4) (end 166.5 90.5) (width 0.15) (layer "F.Cu") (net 21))
 (via (at 166.5 90.5) (size 0.45) (drill 0.2) (layers "F.Cu" "B.Cu") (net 21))
 (via (at 160.7 90.5) (size 0.45) (drill 0.2) (layers "F.Cu" "B.Cu") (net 21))
 (via (at 152.7 90.5) (size 0.45) (drill 0.2) (layers "F.Cu" "B.Cu") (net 21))
 (segment (start 152.7 90.5) (end 166.5 90.5) (width 0.15) (layer "B.Cu") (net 21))
 (segment (start 161.4 97.3) (end 161.2 97.5) (width 0.3) (layer "F.Cu") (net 2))
 (segment (start 153.2 80.3) (end 153.2 82.2) (width 0.15) (layer "F.Cu") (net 2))
 (segment (start 167 89.4) (end 167 91.2) (width 0.15) (layer "F.Cu") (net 2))
 (segment (start 167 53) (end 167 54.9) (width 0.15) (layer "F.Cu") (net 2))
 (segment (start 167 80.3) (end 167 82.2) (width 0.15) (layer "F.Cu") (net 2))
 (segment (start 167 62.4) (end 167 64) (width 0.15) (layer "F.Cu") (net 2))
 (segment (start 153.2 53) (end 153.2 54.9) (width 0.15) (layer "F.Cu") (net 2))
 (segment (start 161.2 97.5) (end 161.2 98.5) (width 0.3) (layer "F.Cu") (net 2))
 (segment (start 167 71.4) (end 167 73.05) (width 0.15) (layer "F.Cu") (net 2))
 (segment (start 153.2 71.2) (end 153.2 73.05) (width 0.15) (layer "F.Cu") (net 2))
 (segment (start 161.4 97.2) (end 161.4 97.3) (width 0.3) (layer "F.Cu") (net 2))
 (segment (start 153.2 62.1) (end 153.2 64) (width 0.15) (layer "F.Cu") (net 2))
 (segment (start 167 43.9) (end 167 45.7) (width 0.15) (layer "F.Cu") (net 2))
 (segment (start 161.4 97.2) (end 161.4 45.7) (width 0.5) (layer "F.Cu") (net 2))
 (segment (start 153.2 43.9) (end 153.2 45.7) (width 0.15) (layer "F.Cu") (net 2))
 (segment (start 153.2 89.4) (end 153.2 91.2) (width 0.15) (layer "F.Cu") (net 2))
 (via (at 167 64) (size 0.45) (drill 0.2) (layers "F.Cu" "B.Cu") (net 2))
 (via (at 167 91.2) (size 0.45) (drill 0.2) (layers "F.Cu" "B.Cu") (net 2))
 (via (at 167 82.2) (size 0.45) (drill 0.2) (layers "F.Cu" "B.Cu") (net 2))
 (via (at 161.4 45.7) (size 0.45) (drill 0.2) (layers "F.Cu" "B.Cu") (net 2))
 (via (at 153.2 45.7) (size 0.45) (drill 0.2) (layers "F.Cu" "B.Cu") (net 2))
 (via (at 153.2 54.9) (size 0.45) (drill 0.2) (layers "F.Cu" "B.Cu") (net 2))
 (via (at 153.2 64) (size 0.45) (drill 0.2) (layers "F.Cu" "B.Cu") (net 2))
 (via (at 167 45.7) (size 0.45) (drill 0.2) (layers "F.Cu" "B.Cu") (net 2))
 (via (at 153.2 82.2) (size 0.45) (drill 0.2) (layers "F.Cu" "B.Cu") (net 2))
 (via (at 161.4 54.9) (size 0.45) (drill 0.2) (layers "F.Cu" "B.Cu") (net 2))
 (via (at 161.4 82.2) (size 0.45) (drill 0.2) (layers "F.Cu" "B.Cu") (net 2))
 (via (at 153.2 91.2) (size 0.45) (drill 0.2) (layers "F.Cu" "B.Cu") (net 2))
 (via (at 161.4 91.2) (size 0.45) (drill 0.2) (layers "F.Cu" "B.Cu") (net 2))
 (via (at 161.4 64) (size 0.45) (drill 0.2) (layers "F.Cu" "B.Cu") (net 2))
 (via (at 161.4 73.05) (size 0.45) (drill 0.2) (layers "F.Cu" "B.Cu") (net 2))
 (via (at 167 73.05) (size 0.45) (drill 0.2) (layers "F.Cu" "B.Cu") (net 2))
 (via (at 153.2 73.05) (size 0.45) (drill 0.2) (layers "F.Cu" "B.Cu") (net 2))
 (via (at 167 54.9) (size 0.45) (drill 0.2) (layers "F.Cu" "B.Cu") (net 2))
 (segment (start 153.2 45.7) (end 167 45.7) (width 0.5) (layer "B.Cu") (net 2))
 (segment (start 153.2 82.2) (end 167 82.2) (width 0.5) (layer "B.Cu") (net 2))
 (segment (start 153.2 64) (end 167 64) (width 0.5) (layer "B.Cu") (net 2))
 (segment (start 153.2 73.05) (end 167 73.05) (width 0.5) (layer "B.Cu") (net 2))
 (segment (start 153.2 54.9) (end 167 54.9) (width 0.5) (layer "B.Cu") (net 2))
 (segment (start 153.2 91.2) (end 167 91.2) (width 0.5) (layer "B.Cu") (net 2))
 (segment (start 169 89.4) (end 169 91.9) (width 0.15) (layer "F.Cu") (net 16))
 (segment (start 169 89.4) (end 169 92.7) (width 0.15) (layer "F.Cu") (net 16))
 (segment (start 169 92.7) (end 168.5 93.2) (width 0.15) (layer "F.Cu") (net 16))
 (segment (start 163.2 93.9) (end 163.2 98.5) (width 0.15) (layer "F.Cu") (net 16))
 (segment (start 168.5 93.2) (end 163.9 93.2) (width 0.15) (layer "F.Cu") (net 16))
 (segment (start 169 43.9) (end 169 89.4) (width 0.15) (layer "F.Cu") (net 16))
 (segment (start 163.9 93.2) (end 163.2 93.9) (width 0.15) (layer "F.Cu") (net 16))
 (segment (start 162.7 93.8) (end 163.35 93.15) (width 0.15) (layer "F.Cu") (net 10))
 (segment (start 163.35 93.15) (end 163.35 47.4) (width 0.15) (layer "F.Cu") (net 10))
 (segment (start 162.7 98.5) (end 162.7 93.8) (width 0.15) (layer "F.Cu") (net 10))
 (segment (start 154.7 43.9) (end 154.7 47.4) (width 0.15) (layer "F.Cu") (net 10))
 (via (at 154.7 47.4) (size 0.45) (drill 0.2) (layers "F.Cu" "B.Cu") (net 10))
 (via (at 163.35 47.4) (size 0.45) (drill 0.2) (layers "F.Cu" "B.Cu") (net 10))
 (segment (start 154.7 47.4) (end 163.35 47.4) (width 0.15) (layer "B.Cu") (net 10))
 (segment (start 168 89.4) (end 168 91.2) (width 0.15) (layer "F.Cu") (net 22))
 (segment (start 162.2 98.5) (end 162.2 99.6) (width 0.15) (layer "F.Cu") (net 22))
 (via (at 162.2 99.6) (size 0.45) (drill 0.2) (layers "F.Cu" "B.Cu") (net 22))
 (via (at 168 91.2) (size 0.45) (drill 0.2) (layers "F.Cu" "B.Cu") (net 22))
 (segment (start 168 92.3) (end 162.2 98.1) (width 0.15) (layer "B.Cu") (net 22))
 (segment (start 162.2 98.1) (end 162.2 99.6) (width 0.15) (layer "B.Cu") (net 22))
 (segment (start 168 91.2) (end 168 92.3) (width 0.15) (layer "B.Cu") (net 22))
 (segment (start 154.2 48.2) (end 154.7 48.7) (width 0.15) (layer "F.Cu") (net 5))
 (segment (start 154.7 48.7) (end 154.7 53) (width 0.15) (layer "F.Cu") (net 5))
 (segment (start 154.2 43.9) (end 154.2 48.2) (width 0.15) (layer "F.Cu") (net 5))
 (segment (start 154.7 57.8) (end 154.7 62.1) (width 0.15) (layer "F.Cu") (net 4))
 (segment (start 154.2 53) (end 154.2 57.3) (width 0.15) (layer "F.Cu") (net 4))
 (segment (start 154.2 57.3) (end 154.7 57.8) (width 0.15) (layer "F.Cu") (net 4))
 (segment (start 154.2 62.1) (end 154.2 66.4) (width 0.15) (layer "F.Cu") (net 26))
 (segment (start 154.2 66.4) (end 154.7 66.9) (width 0.15) (layer "F.Cu") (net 26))
 (segment (start 154.7 66.9) (end 154.7 71.2) (width 0.15) (layer "F.Cu") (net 26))
 (segment (start 154.7 76) (end 154.7 80.3) (width 0.15) (layer "F.Cu") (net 25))
 (segment (start 154.2 75.5) (end 154.7 76) (width 0.15) (layer "F.Cu") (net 25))
 (segment (start 154.2 71.2) (end 154.2 75.5) (width 0.15) (layer "F.Cu") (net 25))
 (segment (start 154.7 85.1) (end 154.7 89.4) (width 0.15) (layer "F.Cu") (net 45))
 (segment (start 154.2 80.3) (end 154.2 84.6) (width 0.15) (layer "F.Cu") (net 45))
 (segment (start 154.2 84.6) (end 154.7 85.1) (width 0.15) (layer "F.Cu") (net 45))
 (segment (start 168.5 43.9) (end 168.5 47.95) (width 0.15) (layer "F.Cu") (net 35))
 (segment (start 162.75 92.9) (end 162.75 47.95) (width 0.15) (layer "F.Cu") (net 35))
 (segment (start 154.2 89.4) (end 154.2 92.9) (width 0.15) (layer "F.Cu") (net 35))
 (via (at 168.5 47.95) (size 0.45) (drill 0.2) (layers "F.Cu" "B.Cu") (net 35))
 (via (at 162.75 92.9) (size 0.45) (drill 0.2) (layers "F.Cu" "B.Cu") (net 35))
 (via (at 154.2 92.9) (size 0.45) (drill 0.2) (layers "F.Cu" "B.Cu") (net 35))
 (via (at 162.75 47.95) (size 0.45) (drill 0.2) (layers "F.Cu" "B.Cu") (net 35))
 (segment (start 154.2 92.9) (end 162.75 92.9) (width 0.15) (layer "B.Cu") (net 35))
 (segment (start 168.5 47.95) (end 162.75 47.95) (width 0.15) (layer "B.Cu") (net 35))
 (segment (start 168 80.3) (end 168 84.6) (width 0.15) (layer "F.Cu") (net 14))
 (segment (start 168 84.6) (end 168.5 85.1) (width 0.15) (layer "F.Cu") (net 14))
 (segment (start 168.5 85.1) (end 168.5 89.4) (width 0.15) (layer "F.Cu") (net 14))
 (segment (start 168 75.6) (end 168.5 76.1) (width 0.15) (layer "F.Cu") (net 15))
 (segment (start 168 71.4) (end 168 75.6) (width 0.15) (layer "F.Cu") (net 15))
 (segment (start 168.5 76.1) (end 168.5 80.3) (width 0.15) (layer "F.Cu") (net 15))
 (segment (start 168 62.4) (end 168 66.65) (width 0.15) (layer "F.Cu") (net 29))
 (segment (start 168 66.65) (end 168.5 67.15) (width 0.15) (layer "F.Cu") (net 29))
 (segment (start 168.5 67.15) (end 168.5 71.4) (width 0.15) (layer "F.Cu") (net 29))
 (segment (start 168 57.45) (end 168.5 57.95) (width 0.15) (layer "F.Cu") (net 38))
 (segment (start 168 53) (end 168 57.45) (width 0.15) (layer "F.Cu") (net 38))
 (segment (start 168.5 57.95) (end 168.5 62.4) (width 0.15) (layer "F.Cu") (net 38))
 (segment (start 168 48.2) (end 168.5 48.7) (width 0.15) (layer "F.Cu") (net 34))
 (segment (start 168 43.9) (end 168 48.2) (width 0.15) (layer "F.Cu") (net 34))
 (segment (start 168.5 48.7) (end 168.5 53) (width 0.15) (layer "F.Cu") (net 34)))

